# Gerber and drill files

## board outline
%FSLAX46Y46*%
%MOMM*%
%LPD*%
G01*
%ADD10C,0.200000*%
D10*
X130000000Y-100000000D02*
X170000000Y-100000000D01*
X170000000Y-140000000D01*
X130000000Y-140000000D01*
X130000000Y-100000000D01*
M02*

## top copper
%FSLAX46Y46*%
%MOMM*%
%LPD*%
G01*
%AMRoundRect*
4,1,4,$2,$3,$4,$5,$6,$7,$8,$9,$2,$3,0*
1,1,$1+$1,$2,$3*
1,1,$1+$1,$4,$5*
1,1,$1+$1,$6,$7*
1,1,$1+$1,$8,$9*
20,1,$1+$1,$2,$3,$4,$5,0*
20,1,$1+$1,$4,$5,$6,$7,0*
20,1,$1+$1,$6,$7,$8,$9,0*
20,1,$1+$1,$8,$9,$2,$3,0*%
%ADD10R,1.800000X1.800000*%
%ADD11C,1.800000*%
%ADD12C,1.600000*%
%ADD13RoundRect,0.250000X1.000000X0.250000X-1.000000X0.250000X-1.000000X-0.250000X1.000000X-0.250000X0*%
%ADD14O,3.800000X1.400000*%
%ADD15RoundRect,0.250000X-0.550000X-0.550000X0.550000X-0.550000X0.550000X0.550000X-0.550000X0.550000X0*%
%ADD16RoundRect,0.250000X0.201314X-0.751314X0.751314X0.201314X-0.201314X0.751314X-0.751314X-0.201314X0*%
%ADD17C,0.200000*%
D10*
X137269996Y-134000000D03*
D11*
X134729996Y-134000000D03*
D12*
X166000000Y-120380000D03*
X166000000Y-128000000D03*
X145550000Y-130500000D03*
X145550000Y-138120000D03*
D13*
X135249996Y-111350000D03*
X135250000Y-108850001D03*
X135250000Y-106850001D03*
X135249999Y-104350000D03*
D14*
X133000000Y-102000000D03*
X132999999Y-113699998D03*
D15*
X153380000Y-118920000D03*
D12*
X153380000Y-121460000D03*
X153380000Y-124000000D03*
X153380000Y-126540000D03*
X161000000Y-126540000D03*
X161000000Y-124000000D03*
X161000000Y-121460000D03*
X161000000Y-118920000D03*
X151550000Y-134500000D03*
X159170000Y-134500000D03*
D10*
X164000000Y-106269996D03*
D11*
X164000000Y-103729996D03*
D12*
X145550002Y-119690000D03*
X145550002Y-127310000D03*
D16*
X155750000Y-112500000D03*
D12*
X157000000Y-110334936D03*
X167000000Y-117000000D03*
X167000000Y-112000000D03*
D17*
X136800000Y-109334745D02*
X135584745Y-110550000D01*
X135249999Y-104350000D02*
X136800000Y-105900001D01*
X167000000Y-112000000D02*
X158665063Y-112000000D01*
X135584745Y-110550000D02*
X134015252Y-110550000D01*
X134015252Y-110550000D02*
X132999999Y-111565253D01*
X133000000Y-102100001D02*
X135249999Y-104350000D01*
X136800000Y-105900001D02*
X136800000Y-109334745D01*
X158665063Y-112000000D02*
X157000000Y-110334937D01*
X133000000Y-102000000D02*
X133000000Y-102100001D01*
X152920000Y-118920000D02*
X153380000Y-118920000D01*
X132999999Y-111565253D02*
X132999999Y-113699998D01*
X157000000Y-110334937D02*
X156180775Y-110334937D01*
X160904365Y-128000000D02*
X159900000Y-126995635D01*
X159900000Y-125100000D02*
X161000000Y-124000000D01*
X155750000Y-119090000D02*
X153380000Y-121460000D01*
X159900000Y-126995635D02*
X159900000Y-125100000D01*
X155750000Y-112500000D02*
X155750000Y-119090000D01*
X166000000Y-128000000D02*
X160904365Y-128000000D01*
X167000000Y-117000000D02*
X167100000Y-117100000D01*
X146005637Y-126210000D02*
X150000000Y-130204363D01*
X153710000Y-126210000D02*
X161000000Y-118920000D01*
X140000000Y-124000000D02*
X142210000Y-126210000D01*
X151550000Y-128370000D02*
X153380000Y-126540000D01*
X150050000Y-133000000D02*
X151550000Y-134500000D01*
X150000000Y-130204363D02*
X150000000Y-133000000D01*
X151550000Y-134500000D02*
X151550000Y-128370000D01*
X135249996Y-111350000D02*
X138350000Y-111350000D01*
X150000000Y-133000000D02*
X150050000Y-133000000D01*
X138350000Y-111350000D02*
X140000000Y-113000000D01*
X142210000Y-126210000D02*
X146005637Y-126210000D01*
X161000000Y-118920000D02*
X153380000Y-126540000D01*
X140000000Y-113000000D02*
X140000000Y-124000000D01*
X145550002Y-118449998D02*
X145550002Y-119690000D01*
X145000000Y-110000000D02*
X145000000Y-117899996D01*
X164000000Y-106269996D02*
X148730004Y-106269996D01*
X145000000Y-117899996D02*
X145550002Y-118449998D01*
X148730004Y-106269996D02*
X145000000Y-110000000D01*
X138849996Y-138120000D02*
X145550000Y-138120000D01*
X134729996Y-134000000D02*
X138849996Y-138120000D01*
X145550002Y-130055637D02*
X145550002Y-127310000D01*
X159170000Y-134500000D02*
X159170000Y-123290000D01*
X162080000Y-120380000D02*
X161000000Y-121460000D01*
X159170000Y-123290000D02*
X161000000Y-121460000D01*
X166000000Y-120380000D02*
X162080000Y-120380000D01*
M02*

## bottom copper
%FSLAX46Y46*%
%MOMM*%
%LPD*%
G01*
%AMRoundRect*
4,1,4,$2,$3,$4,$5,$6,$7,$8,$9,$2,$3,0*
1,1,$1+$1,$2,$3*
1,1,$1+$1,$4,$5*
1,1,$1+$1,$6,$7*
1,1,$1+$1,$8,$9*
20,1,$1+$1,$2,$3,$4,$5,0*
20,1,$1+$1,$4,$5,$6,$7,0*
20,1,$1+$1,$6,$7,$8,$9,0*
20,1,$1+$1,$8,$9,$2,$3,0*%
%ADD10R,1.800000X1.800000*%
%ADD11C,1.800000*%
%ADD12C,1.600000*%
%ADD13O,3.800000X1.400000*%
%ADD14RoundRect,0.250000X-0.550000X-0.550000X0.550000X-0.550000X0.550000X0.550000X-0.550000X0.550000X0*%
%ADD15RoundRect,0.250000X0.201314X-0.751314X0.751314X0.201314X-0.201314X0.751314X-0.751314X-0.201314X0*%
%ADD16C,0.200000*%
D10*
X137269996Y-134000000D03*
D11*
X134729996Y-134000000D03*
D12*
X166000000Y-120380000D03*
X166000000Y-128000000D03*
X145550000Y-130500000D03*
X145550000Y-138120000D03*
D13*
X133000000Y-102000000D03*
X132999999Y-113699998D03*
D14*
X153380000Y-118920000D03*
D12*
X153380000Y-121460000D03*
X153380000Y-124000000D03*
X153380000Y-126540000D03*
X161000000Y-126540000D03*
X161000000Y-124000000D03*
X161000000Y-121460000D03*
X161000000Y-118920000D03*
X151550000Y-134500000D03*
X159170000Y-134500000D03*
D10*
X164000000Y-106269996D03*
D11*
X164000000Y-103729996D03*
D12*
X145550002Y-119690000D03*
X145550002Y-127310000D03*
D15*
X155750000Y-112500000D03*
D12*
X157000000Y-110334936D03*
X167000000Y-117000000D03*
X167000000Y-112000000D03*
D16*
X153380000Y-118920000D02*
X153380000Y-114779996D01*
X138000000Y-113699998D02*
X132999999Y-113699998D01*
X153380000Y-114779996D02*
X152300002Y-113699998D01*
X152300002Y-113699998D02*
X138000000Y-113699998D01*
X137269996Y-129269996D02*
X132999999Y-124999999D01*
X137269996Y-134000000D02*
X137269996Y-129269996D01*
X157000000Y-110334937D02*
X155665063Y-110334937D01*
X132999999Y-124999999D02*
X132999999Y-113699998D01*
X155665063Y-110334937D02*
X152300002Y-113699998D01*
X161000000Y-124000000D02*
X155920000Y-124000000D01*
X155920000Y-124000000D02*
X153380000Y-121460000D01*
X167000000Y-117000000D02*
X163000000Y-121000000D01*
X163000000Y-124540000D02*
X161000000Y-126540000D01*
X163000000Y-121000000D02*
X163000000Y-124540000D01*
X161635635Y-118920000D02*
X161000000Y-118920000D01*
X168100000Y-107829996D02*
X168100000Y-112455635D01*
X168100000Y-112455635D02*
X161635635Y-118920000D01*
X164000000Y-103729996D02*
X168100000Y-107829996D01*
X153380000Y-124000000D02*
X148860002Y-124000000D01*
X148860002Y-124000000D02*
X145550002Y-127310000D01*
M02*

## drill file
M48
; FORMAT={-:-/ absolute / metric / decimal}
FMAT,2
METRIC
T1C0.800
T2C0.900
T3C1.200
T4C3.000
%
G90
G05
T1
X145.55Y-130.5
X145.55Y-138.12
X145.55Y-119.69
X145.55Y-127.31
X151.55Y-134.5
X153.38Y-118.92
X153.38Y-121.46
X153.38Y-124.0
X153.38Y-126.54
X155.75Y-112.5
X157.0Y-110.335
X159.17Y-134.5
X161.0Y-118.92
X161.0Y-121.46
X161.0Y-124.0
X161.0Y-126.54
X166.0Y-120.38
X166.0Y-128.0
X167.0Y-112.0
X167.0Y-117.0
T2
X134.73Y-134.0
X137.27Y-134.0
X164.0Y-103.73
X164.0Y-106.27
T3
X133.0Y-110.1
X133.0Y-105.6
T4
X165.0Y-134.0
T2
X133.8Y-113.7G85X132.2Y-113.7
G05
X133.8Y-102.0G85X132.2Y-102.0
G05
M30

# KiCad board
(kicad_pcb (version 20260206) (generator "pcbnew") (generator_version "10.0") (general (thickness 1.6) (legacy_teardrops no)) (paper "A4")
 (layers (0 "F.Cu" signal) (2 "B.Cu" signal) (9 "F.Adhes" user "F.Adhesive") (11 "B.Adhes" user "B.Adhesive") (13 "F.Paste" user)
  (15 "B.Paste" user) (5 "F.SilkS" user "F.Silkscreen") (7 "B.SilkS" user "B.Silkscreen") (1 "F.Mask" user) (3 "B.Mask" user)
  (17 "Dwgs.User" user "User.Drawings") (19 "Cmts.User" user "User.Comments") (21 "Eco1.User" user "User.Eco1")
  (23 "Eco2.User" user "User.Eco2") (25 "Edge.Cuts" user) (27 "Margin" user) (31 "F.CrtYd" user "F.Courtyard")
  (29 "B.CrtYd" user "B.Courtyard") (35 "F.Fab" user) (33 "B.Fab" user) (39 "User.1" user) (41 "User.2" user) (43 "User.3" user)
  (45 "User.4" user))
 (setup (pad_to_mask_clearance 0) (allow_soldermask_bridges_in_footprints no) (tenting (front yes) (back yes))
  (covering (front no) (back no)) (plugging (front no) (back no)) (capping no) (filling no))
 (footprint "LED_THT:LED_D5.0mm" (layer "F.Cu") (at 137.269996 134 180)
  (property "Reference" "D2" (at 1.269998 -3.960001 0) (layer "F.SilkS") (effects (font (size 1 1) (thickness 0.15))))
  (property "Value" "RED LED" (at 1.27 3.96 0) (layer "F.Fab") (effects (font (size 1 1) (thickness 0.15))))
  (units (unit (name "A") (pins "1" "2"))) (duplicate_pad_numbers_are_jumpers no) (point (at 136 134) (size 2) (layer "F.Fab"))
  (pad "1" thru_hole rect (at 0 0 180) (size 1.8 1.8) (drill 0.9) (layers "*.Cu" "*.Mask") (remove_unused_layers no) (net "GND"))
  (pad "2" thru_hole circle (at 2.54 0 180) (size 1.8 1.8) (drill 0.9) (layers "*.Cu" "*.Mask") (remove_unused_layers no) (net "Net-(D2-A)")))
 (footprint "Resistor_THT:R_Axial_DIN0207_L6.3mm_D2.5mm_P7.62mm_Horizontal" (layer "F.Cu") (at 166 120.38 -90)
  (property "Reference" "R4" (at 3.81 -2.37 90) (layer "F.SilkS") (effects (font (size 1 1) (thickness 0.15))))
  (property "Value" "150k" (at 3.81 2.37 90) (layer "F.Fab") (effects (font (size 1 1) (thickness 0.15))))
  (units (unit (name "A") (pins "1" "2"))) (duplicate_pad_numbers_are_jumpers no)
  (pad "1" thru_hole circle (at 0 0 270) (size 1.6 1.6) (drill 0.8) (layers "*.Cu" "*.Mask") (remove_unused_layers no)
   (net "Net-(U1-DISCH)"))
  (pad "2" thru_hole circle (at 7.62 0 270) (size 1.6 1.6) (drill 0.8) (layers "*.Cu" "*.Mask") (remove_unused_layers no)
   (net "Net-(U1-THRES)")))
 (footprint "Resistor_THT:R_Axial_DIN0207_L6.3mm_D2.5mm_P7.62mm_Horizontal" (layer "F.Cu") (at 145.55 130.5 -90)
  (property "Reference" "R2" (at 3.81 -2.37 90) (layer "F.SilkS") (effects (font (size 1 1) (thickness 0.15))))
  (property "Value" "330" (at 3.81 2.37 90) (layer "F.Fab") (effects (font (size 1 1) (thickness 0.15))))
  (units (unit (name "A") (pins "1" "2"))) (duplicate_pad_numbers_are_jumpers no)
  (pad "1" thru_hole circle (at 0 0 270) (size 1.6 1.6) (drill 0.8) (layers "*.Cu" "*.Mask") (remove_unused_layers no) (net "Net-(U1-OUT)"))
  (pad "2" thru_hole circle (at 7.62 0 270) (size 1.6 1.6) (drill 0.8) (layers "*.Cu" "*.Mask") (remove_unused_layers no) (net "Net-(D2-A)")))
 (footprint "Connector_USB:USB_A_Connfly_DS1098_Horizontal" (layer "F.Cu") (at 124.7 107.850001 180)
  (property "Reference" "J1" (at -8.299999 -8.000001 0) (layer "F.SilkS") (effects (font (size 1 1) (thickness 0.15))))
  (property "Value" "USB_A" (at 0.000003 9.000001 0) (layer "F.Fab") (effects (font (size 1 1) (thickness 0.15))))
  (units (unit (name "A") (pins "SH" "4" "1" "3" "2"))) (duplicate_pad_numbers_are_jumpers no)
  (pad "" np_thru_hole circle (at -8.300001 2.249997 180) (size 1.2 1.2) (drill 1.2) (layers "*.Mask"))
  (pad "" np_thru_hole circle (at -8.3 -2.250002 180) (size 1.2 1.2) (drill 1.2) (layers "*.Mask"))
  (pad "1" smd roundrect (at -10.549996 -3.499999 180) (size 2.5 1) (layers "F.Cu" "F.Mask" "F.Paste") (roundrect_rratio 0.25)
   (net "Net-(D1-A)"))
  (pad "2" smd roundrect (at -10.55 -1 180) (size 2.5 1) (layers "F.Cu" "F.Mask" "F.Paste") (roundrect_rratio 0.25)
   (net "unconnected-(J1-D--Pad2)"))
  (pad "3" smd roundrect (at -10.55 1 180) (size 2.5 1) (layers "F.Cu" "F.Mask" "F.Paste") (roundrect_rratio 0.25)
   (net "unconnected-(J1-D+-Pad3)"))
  (pad "4" smd roundrect (at -10.549999 3.500001 180) (size 2.5 1) (layers "F.Cu" "F.Mask" "F.Paste") (roundrect_rratio 0.25) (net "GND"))
  (pad "SH" thru_hole oval (at -8.3 5.850001 180) (size 3.8 1.4) (drill oval 2.5 0.9) (layers "*.Cu" "*.Mask") (remove_unused_layers no)
   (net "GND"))
  (pad "SH" thru_hole oval (at -8.299999 -5.849997 180) (size 3.8 1.4) (drill oval 2.5 0.9) (layers "*.Cu" "*.Mask")
   (remove_unused_layers no) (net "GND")))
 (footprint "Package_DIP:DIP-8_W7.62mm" (layer "F.Cu") (at 153.38 118.92)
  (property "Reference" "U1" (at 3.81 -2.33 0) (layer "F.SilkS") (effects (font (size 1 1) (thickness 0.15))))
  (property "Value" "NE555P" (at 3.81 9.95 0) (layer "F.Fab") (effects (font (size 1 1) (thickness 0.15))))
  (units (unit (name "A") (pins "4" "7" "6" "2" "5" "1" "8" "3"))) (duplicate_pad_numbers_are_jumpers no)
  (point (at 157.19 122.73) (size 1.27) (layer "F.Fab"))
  (pad "1" thru_hole roundrect (at 0 0) (size 1.6 1.6) (drill 0.8) (layers "*.Cu" "*.Mask") (remove_unused_layers no)
   (roundrect_rratio 0.15625) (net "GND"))
  (pad "2" thru_hole circle (at 0 2.54) (size 1.6 1.6) (drill 0.8) (layers "*.Cu" "*.Mask") (remove_unused_layers no) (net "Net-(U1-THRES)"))
  (pad "3" thru_hole circle (at 0 5.08) (size 1.6 1.6) (drill 0.8) (layers "*.Cu" "*.Mask") (remove_unused_layers no) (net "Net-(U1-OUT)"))
  (pad "4" thru_hole circle (at 0 7.62) (size 1.6 1.6) (drill 0.8) (layers "*.Cu" "*.Mask") (remove_unused_layers no) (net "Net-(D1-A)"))
  (pad "5" thru_hole circle (at 7.62 7.62) (size 1.6 1.6) (drill 0.8) (layers "*.Cu" "*.Mask") (remove_unused_layers no)
   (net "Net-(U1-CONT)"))
  (pad "6" thru_hole circle (at 7.62 5.08) (size 1.6 1.6) (drill 0.8) (layers "*.Cu" "*.Mask") (remove_unused_layers no)
   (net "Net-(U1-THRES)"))
  (pad "7" thru_hole circle (at 7.62 2.54) (size 1.6 1.6) (drill 0.8) (layers "*.Cu" "*.Mask") (remove_unused_layers no)
   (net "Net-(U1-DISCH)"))
  (pad "8" thru_hole circle (at 7.62 0) (size 1.6 1.6) (drill 0.8) (layers "*.Cu" "*.Mask") (remove_unused_layers no) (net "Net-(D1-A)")))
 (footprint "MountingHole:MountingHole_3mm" (layer "F.Cu") (at 165 134)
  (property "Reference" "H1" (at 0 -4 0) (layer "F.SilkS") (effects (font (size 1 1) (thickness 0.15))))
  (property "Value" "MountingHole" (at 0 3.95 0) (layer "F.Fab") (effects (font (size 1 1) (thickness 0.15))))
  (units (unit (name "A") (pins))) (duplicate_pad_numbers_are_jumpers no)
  (pad "" np_thru_hole circle (at 0 0) (size 3 3) (drill 3) (layers "*.Cu" "*.Mask")))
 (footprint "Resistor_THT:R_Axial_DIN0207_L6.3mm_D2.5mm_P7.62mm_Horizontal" (layer "F.Cu") (at 151.55 134.5)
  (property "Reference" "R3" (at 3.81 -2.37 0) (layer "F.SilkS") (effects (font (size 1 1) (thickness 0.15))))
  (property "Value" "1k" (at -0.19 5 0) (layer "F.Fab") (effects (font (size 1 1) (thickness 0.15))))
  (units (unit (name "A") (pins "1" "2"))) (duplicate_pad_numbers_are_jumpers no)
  (pad "1" thru_hole circle (at 0 0) (size 1.6 1.6) (drill 0.8) (layers "*.Cu" "*.Mask") (remove_unused_layers no) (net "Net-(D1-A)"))
  (pad "2" thru_hole circle (at 7.62 0) (size 1.6 1.6) (drill 0.8) (layers "*.Cu" "*.Mask") (remove_unused_layers no) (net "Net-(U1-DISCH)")))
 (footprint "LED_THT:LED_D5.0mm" (layer "F.Cu") (at 164 106.269996 90)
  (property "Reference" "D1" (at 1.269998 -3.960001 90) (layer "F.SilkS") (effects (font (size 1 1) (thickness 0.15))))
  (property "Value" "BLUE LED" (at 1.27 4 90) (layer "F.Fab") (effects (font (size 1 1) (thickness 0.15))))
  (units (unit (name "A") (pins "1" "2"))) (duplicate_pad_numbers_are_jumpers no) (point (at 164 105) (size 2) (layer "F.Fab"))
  (pad "1" thru_hole rect (at 0 0 90) (size 1.8 1.8) (drill 0.9) (layers "*.Cu" "*.Mask") (remove_unused_layers no) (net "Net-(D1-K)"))
  (pad "2" thru_hole circle (at 2.54 0 90) (size 1.8 1.8) (drill 0.9) (layers "*.Cu" "*.Mask") (remove_unused_layers no) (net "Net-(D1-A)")))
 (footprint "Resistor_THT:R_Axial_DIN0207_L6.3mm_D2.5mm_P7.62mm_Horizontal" (layer "F.Cu") (at 145.550002 119.69 -90)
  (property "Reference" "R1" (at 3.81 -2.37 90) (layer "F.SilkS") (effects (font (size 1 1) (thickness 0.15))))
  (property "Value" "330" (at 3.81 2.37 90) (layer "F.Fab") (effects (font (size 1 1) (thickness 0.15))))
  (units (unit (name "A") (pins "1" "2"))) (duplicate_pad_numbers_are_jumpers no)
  (pad "1" thru_hole circle (at 0 0 270) (size 1.6 1.6) (drill 0.8) (layers "*.Cu" "*.Mask") (remove_unused_layers no) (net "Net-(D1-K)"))
  (pad "2" thru_hole circle (at 7.62 0 270) (size 1.6 1.6) (drill 0.8) (layers "*.Cu" "*.Mask") (remove_unused_layers no)
   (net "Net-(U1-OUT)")))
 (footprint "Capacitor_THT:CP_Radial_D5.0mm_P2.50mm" (layer "F.Cu") (at 155.75 112.5 60)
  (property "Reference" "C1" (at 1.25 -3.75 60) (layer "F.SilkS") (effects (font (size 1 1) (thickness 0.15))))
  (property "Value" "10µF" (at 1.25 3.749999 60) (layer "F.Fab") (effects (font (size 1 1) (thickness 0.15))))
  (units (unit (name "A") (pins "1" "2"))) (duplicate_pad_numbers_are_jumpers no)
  (pad "1" thru_hole roundrect (at 0 0 60) (size 1.6 1.6) (drill 0.8) (layers "*.Cu" "*.Mask") (remove_unused_layers no)
   (roundrect_rratio 0.15625) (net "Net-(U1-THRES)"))
  (pad "2" thru_hole circle (at 2.5 0 60) (size 1.6 1.6) (drill 0.8) (layers "*.Cu" "*.Mask") (remove_unused_layers no) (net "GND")))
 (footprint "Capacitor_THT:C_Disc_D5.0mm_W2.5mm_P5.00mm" (layer "F.Cu") (at 167 117 90)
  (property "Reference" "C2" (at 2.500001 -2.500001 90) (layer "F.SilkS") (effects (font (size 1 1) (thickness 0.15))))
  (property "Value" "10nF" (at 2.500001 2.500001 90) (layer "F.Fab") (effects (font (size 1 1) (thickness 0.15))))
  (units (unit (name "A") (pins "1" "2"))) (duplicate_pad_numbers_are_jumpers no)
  (pad "1" thru_hole circle (at 0 0 90) (size 1.6 1.6) (drill 0.8) (layers "*.Cu" "*.Mask") (remove_unused_layers no) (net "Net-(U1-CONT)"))
  (pad "2" thru_hole circle (at 5 0 90) (size 1.6 1.6) (drill 0.8) (layers "*.Cu" "*.Mask") (remove_unused_layers no) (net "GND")))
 (gr_rect (start 130 100) (end 170 140) (stroke (width 0.2) (type default)) (fill no) (layer "Edge.Cuts"))
 (segment (start 136.8 109.334745) (end 135.584745 110.55) (width 0.2) (layer "F.Cu") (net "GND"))
 (segment (start 135.249999 104.35) (end 136.8 105.900001) (width 0.2) (layer "F.Cu") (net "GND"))
 (segment (start 167 112) (end 158.665063 112) (width 0.2) (layer "F.Cu") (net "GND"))
 (segment (start 135.584745 110.55) (end 134.015252 110.55) (width 0.2) (layer "F.Cu") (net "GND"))
 (segment (start 134.015252 110.55) (end 132.999999 111.565253) (width 0.2) (layer "F.Cu") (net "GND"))
 (segment (start 133 102.100001) (end 135.249999 104.35) (width 0.2) (layer "F.Cu") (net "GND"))
 (segment (start 136.8 105.900001) (end 136.8 109.334745) (width 0.2) (layer "F.Cu") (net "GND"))
 (segment (start 158.665063 112) (end 157 110.334937) (width 0.2) (layer "F.Cu") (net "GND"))
 (segment (start 133 102) (end 133 102.100001) (width 0.2) (layer "F.Cu") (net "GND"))
 (segment (start 152.92 118.92) (end 153.38 118.92) (width 0.2) (layer "F.Cu") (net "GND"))
 (segment (start 132.999999 111.565253) (end 132.999999 113.699998) (width 0.2) (layer "F.Cu") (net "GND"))
 (segment (start 157 110.334937) (end 156.180775 110.334937) (width 0.2) (layer "F.Cu") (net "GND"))
 (segment (start 153.38 118.92) (end 153.38 114.779996) (width 0.2) (layer "B.Cu") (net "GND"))
 (segment (start 138 113.699998) (end 132.999999 113.699998) (width 0.2) (layer "B.Cu") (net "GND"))
 (segment (start 153.38 114.779996) (end 152.300002 113.699998) (width 0.2) (layer "B.Cu") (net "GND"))
 (segment (start 152.300002 113.699998) (end 138 113.699998) (width 0.2) (layer "B.Cu") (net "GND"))
 (segment (start 137.269996 129.269996) (end 132.999999 124.999999) (width 0.2) (layer "B.Cu") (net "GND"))
 (segment (start 137.269996 134) (end 137.269996 129.269996) (width 0.2) (layer "B.Cu") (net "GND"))
 (segment (start 157 110.334937) (end 155.665063 110.334937) (width 0.2) (layer "B.Cu") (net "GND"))
 (segment (start 132.999999 124.999999) (end 132.999999 113.699998) (width 0.2) (layer "B.Cu") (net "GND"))
 (segment (start 155.665063 110.334937) (end 152.300002 113.699998) (width 0.2) (layer "B.Cu") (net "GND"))
 (segment (start 160.904365 128) (end 159.9 126.995635) (width 0.2) (layer "F.Cu") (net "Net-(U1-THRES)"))
 (segment (start 159.9 125.1) (end 161 124) (width 0.2) (layer "F.Cu") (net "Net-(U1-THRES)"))
 (segment (start 155.75 119.09) (end 153.38 121.46) (width 0.2) (layer "F.Cu") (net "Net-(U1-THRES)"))
 (segment (start 159.9 126.995635) (end 159.9 125.1) (width 0.2) (layer "F.Cu") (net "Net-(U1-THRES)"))
 (segment (start 155.75 112.5) (end 155.75 119.09) (width 0.2) (layer "F.Cu") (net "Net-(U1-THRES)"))
 (segment (start 166 128) (end 160.904365 128) (width 0.2) (layer "F.Cu") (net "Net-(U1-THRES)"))
 (segment (start 161 124) (end 155.92 124) (width 0.2) (layer "B.Cu") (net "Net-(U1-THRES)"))
 (segment (start 155.92 124) (end 153.38 121.46) (width 0.2) (layer "B.Cu") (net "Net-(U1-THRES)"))
 (segment (start 167 117) (end 167.1 117.1) (width 0.2) (layer "F.Cu") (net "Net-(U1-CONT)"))
 (segment (start 167 117) (end 163 121) (width 0.2) (layer "B.Cu") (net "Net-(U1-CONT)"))
 (segment (start 163 124.54) (end 161 126.54) (width 0.2) (layer "B.Cu") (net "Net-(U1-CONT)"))
 (segment (start 163 121) (end 163 124.54) (width 0.2) (layer "B.Cu") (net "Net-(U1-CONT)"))
 (segment (start 146.005637 126.21) (end 150 130.204363) (width 0.2) (layer "F.Cu") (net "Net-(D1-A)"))
 (segment (start 153.71 126.21) (end 161 118.92) (width 0.2) (layer "F.Cu") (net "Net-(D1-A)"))
 (segment (start 140 124) (end 142.21 126.21) (width 0.2) (layer "F.Cu") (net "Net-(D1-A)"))
 (segment (start 151.55 128.37) (end 153.38 126.54) (width 0.2) (layer "F.Cu") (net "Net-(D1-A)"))
 (segment (start 150.05 133) (end 151.55 134.5) (width 0.2) (layer "F.Cu") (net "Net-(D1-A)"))
 (segment (start 150 130.204363) (end 150 133) (width 0.2) (layer "F.Cu") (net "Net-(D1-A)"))
 (segment (start 151.55 134.5) (end 151.55 128.37) (width 0.2) (layer "F.Cu") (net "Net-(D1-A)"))
 (segment (start 135.249996 111.35) (end 138.35 111.35) (width 0.2) (layer "F.Cu") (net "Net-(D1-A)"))
 (segment (start 150 133) (end 150.05 133) (width 0.2) (layer "F.Cu") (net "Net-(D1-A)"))
 (segment (start 138.35 111.35) (end 140 113) (width 0.2) (layer "F.Cu") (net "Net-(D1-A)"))
 (segment (start 142.21 126.21) (end 146.005637 126.21) (width 0.2) (layer "F.Cu") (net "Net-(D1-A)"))
 (segment (start 161 118.92) (end 153.38 126.54) (width 0.2) (layer "F.Cu") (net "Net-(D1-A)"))
 (segment (start 140 113) (end 140 124) (width 0.2) (layer "F.Cu") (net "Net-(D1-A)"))
 (segment (start 161.635635 118.92) (end 161 118.92) (width 0.2) (layer "B.Cu") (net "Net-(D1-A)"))
 (segment (start 168.1 107.829996) (end 168.1 112.455635) (width 0.2) (layer "B.Cu") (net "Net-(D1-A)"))
 (segment (start 168.1 112.455635) (end 161.635635 118.92) (width 0.2) (layer "B.Cu") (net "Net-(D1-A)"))
 (segment (start 164 103.729996) (end 168.1 107.829996) (width 0.2) (layer "B.Cu") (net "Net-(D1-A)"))
 (segment (start 145.550002 118.449998) (end 145.550002 119.69) (width 0.2) (layer "F.Cu") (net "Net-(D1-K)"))
 (segment (start 145 110) (end 145 117.899996) (width 0.2) (layer "F.Cu") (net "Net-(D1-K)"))
 (segment (start 164 106.269996) (end 148.730004 106.269996) (width 0.2) (layer "F.Cu") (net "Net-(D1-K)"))
 (segment (start 145 117.899996) (end 145.550002 118.449998) (width 0.2) (layer "F.Cu") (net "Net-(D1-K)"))
 (segment (start 148.730004 106.269996) (end 145 110) (width 0.2) (layer "F.Cu") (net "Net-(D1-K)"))
 (segment (start 138.849996 138.12) (end 145.55 138.12) (width 0.2) (layer "F.Cu") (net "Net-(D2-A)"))
 (segment (start 134.729996 134) (end 138.849996 138.12) (width 0.2) (layer "F.Cu") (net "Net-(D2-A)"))
 (segment (start 145.550002 130.055637) (end 145.550002 127.31) (width 0.2) (layer "F.Cu") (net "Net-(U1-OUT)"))
 (segment (start 153.38 124) (end 148.860002 124) (width 0.2) (layer "B.Cu") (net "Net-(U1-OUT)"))
 (segment (start 148.860002 124) (end 145.550002 127.31) (width 0.2) (layer "B.Cu") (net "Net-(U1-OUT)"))
 (segment (start 159.17 134.5) (end 159.17 123.29) (width 0.2) (layer "F.Cu") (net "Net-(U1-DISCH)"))
 (segment (start 162.08 120.38) (end 161 121.46) (width 0.2) (layer "F.Cu") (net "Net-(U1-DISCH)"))
 (segment (start 159.17 123.29) (end 161 121.46) (width 0.2) (layer "F.Cu") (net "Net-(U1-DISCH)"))
 (segment (start 166 120.38) (end 162.08 120.38) (width 0.2) (layer "F.Cu") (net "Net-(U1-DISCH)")))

